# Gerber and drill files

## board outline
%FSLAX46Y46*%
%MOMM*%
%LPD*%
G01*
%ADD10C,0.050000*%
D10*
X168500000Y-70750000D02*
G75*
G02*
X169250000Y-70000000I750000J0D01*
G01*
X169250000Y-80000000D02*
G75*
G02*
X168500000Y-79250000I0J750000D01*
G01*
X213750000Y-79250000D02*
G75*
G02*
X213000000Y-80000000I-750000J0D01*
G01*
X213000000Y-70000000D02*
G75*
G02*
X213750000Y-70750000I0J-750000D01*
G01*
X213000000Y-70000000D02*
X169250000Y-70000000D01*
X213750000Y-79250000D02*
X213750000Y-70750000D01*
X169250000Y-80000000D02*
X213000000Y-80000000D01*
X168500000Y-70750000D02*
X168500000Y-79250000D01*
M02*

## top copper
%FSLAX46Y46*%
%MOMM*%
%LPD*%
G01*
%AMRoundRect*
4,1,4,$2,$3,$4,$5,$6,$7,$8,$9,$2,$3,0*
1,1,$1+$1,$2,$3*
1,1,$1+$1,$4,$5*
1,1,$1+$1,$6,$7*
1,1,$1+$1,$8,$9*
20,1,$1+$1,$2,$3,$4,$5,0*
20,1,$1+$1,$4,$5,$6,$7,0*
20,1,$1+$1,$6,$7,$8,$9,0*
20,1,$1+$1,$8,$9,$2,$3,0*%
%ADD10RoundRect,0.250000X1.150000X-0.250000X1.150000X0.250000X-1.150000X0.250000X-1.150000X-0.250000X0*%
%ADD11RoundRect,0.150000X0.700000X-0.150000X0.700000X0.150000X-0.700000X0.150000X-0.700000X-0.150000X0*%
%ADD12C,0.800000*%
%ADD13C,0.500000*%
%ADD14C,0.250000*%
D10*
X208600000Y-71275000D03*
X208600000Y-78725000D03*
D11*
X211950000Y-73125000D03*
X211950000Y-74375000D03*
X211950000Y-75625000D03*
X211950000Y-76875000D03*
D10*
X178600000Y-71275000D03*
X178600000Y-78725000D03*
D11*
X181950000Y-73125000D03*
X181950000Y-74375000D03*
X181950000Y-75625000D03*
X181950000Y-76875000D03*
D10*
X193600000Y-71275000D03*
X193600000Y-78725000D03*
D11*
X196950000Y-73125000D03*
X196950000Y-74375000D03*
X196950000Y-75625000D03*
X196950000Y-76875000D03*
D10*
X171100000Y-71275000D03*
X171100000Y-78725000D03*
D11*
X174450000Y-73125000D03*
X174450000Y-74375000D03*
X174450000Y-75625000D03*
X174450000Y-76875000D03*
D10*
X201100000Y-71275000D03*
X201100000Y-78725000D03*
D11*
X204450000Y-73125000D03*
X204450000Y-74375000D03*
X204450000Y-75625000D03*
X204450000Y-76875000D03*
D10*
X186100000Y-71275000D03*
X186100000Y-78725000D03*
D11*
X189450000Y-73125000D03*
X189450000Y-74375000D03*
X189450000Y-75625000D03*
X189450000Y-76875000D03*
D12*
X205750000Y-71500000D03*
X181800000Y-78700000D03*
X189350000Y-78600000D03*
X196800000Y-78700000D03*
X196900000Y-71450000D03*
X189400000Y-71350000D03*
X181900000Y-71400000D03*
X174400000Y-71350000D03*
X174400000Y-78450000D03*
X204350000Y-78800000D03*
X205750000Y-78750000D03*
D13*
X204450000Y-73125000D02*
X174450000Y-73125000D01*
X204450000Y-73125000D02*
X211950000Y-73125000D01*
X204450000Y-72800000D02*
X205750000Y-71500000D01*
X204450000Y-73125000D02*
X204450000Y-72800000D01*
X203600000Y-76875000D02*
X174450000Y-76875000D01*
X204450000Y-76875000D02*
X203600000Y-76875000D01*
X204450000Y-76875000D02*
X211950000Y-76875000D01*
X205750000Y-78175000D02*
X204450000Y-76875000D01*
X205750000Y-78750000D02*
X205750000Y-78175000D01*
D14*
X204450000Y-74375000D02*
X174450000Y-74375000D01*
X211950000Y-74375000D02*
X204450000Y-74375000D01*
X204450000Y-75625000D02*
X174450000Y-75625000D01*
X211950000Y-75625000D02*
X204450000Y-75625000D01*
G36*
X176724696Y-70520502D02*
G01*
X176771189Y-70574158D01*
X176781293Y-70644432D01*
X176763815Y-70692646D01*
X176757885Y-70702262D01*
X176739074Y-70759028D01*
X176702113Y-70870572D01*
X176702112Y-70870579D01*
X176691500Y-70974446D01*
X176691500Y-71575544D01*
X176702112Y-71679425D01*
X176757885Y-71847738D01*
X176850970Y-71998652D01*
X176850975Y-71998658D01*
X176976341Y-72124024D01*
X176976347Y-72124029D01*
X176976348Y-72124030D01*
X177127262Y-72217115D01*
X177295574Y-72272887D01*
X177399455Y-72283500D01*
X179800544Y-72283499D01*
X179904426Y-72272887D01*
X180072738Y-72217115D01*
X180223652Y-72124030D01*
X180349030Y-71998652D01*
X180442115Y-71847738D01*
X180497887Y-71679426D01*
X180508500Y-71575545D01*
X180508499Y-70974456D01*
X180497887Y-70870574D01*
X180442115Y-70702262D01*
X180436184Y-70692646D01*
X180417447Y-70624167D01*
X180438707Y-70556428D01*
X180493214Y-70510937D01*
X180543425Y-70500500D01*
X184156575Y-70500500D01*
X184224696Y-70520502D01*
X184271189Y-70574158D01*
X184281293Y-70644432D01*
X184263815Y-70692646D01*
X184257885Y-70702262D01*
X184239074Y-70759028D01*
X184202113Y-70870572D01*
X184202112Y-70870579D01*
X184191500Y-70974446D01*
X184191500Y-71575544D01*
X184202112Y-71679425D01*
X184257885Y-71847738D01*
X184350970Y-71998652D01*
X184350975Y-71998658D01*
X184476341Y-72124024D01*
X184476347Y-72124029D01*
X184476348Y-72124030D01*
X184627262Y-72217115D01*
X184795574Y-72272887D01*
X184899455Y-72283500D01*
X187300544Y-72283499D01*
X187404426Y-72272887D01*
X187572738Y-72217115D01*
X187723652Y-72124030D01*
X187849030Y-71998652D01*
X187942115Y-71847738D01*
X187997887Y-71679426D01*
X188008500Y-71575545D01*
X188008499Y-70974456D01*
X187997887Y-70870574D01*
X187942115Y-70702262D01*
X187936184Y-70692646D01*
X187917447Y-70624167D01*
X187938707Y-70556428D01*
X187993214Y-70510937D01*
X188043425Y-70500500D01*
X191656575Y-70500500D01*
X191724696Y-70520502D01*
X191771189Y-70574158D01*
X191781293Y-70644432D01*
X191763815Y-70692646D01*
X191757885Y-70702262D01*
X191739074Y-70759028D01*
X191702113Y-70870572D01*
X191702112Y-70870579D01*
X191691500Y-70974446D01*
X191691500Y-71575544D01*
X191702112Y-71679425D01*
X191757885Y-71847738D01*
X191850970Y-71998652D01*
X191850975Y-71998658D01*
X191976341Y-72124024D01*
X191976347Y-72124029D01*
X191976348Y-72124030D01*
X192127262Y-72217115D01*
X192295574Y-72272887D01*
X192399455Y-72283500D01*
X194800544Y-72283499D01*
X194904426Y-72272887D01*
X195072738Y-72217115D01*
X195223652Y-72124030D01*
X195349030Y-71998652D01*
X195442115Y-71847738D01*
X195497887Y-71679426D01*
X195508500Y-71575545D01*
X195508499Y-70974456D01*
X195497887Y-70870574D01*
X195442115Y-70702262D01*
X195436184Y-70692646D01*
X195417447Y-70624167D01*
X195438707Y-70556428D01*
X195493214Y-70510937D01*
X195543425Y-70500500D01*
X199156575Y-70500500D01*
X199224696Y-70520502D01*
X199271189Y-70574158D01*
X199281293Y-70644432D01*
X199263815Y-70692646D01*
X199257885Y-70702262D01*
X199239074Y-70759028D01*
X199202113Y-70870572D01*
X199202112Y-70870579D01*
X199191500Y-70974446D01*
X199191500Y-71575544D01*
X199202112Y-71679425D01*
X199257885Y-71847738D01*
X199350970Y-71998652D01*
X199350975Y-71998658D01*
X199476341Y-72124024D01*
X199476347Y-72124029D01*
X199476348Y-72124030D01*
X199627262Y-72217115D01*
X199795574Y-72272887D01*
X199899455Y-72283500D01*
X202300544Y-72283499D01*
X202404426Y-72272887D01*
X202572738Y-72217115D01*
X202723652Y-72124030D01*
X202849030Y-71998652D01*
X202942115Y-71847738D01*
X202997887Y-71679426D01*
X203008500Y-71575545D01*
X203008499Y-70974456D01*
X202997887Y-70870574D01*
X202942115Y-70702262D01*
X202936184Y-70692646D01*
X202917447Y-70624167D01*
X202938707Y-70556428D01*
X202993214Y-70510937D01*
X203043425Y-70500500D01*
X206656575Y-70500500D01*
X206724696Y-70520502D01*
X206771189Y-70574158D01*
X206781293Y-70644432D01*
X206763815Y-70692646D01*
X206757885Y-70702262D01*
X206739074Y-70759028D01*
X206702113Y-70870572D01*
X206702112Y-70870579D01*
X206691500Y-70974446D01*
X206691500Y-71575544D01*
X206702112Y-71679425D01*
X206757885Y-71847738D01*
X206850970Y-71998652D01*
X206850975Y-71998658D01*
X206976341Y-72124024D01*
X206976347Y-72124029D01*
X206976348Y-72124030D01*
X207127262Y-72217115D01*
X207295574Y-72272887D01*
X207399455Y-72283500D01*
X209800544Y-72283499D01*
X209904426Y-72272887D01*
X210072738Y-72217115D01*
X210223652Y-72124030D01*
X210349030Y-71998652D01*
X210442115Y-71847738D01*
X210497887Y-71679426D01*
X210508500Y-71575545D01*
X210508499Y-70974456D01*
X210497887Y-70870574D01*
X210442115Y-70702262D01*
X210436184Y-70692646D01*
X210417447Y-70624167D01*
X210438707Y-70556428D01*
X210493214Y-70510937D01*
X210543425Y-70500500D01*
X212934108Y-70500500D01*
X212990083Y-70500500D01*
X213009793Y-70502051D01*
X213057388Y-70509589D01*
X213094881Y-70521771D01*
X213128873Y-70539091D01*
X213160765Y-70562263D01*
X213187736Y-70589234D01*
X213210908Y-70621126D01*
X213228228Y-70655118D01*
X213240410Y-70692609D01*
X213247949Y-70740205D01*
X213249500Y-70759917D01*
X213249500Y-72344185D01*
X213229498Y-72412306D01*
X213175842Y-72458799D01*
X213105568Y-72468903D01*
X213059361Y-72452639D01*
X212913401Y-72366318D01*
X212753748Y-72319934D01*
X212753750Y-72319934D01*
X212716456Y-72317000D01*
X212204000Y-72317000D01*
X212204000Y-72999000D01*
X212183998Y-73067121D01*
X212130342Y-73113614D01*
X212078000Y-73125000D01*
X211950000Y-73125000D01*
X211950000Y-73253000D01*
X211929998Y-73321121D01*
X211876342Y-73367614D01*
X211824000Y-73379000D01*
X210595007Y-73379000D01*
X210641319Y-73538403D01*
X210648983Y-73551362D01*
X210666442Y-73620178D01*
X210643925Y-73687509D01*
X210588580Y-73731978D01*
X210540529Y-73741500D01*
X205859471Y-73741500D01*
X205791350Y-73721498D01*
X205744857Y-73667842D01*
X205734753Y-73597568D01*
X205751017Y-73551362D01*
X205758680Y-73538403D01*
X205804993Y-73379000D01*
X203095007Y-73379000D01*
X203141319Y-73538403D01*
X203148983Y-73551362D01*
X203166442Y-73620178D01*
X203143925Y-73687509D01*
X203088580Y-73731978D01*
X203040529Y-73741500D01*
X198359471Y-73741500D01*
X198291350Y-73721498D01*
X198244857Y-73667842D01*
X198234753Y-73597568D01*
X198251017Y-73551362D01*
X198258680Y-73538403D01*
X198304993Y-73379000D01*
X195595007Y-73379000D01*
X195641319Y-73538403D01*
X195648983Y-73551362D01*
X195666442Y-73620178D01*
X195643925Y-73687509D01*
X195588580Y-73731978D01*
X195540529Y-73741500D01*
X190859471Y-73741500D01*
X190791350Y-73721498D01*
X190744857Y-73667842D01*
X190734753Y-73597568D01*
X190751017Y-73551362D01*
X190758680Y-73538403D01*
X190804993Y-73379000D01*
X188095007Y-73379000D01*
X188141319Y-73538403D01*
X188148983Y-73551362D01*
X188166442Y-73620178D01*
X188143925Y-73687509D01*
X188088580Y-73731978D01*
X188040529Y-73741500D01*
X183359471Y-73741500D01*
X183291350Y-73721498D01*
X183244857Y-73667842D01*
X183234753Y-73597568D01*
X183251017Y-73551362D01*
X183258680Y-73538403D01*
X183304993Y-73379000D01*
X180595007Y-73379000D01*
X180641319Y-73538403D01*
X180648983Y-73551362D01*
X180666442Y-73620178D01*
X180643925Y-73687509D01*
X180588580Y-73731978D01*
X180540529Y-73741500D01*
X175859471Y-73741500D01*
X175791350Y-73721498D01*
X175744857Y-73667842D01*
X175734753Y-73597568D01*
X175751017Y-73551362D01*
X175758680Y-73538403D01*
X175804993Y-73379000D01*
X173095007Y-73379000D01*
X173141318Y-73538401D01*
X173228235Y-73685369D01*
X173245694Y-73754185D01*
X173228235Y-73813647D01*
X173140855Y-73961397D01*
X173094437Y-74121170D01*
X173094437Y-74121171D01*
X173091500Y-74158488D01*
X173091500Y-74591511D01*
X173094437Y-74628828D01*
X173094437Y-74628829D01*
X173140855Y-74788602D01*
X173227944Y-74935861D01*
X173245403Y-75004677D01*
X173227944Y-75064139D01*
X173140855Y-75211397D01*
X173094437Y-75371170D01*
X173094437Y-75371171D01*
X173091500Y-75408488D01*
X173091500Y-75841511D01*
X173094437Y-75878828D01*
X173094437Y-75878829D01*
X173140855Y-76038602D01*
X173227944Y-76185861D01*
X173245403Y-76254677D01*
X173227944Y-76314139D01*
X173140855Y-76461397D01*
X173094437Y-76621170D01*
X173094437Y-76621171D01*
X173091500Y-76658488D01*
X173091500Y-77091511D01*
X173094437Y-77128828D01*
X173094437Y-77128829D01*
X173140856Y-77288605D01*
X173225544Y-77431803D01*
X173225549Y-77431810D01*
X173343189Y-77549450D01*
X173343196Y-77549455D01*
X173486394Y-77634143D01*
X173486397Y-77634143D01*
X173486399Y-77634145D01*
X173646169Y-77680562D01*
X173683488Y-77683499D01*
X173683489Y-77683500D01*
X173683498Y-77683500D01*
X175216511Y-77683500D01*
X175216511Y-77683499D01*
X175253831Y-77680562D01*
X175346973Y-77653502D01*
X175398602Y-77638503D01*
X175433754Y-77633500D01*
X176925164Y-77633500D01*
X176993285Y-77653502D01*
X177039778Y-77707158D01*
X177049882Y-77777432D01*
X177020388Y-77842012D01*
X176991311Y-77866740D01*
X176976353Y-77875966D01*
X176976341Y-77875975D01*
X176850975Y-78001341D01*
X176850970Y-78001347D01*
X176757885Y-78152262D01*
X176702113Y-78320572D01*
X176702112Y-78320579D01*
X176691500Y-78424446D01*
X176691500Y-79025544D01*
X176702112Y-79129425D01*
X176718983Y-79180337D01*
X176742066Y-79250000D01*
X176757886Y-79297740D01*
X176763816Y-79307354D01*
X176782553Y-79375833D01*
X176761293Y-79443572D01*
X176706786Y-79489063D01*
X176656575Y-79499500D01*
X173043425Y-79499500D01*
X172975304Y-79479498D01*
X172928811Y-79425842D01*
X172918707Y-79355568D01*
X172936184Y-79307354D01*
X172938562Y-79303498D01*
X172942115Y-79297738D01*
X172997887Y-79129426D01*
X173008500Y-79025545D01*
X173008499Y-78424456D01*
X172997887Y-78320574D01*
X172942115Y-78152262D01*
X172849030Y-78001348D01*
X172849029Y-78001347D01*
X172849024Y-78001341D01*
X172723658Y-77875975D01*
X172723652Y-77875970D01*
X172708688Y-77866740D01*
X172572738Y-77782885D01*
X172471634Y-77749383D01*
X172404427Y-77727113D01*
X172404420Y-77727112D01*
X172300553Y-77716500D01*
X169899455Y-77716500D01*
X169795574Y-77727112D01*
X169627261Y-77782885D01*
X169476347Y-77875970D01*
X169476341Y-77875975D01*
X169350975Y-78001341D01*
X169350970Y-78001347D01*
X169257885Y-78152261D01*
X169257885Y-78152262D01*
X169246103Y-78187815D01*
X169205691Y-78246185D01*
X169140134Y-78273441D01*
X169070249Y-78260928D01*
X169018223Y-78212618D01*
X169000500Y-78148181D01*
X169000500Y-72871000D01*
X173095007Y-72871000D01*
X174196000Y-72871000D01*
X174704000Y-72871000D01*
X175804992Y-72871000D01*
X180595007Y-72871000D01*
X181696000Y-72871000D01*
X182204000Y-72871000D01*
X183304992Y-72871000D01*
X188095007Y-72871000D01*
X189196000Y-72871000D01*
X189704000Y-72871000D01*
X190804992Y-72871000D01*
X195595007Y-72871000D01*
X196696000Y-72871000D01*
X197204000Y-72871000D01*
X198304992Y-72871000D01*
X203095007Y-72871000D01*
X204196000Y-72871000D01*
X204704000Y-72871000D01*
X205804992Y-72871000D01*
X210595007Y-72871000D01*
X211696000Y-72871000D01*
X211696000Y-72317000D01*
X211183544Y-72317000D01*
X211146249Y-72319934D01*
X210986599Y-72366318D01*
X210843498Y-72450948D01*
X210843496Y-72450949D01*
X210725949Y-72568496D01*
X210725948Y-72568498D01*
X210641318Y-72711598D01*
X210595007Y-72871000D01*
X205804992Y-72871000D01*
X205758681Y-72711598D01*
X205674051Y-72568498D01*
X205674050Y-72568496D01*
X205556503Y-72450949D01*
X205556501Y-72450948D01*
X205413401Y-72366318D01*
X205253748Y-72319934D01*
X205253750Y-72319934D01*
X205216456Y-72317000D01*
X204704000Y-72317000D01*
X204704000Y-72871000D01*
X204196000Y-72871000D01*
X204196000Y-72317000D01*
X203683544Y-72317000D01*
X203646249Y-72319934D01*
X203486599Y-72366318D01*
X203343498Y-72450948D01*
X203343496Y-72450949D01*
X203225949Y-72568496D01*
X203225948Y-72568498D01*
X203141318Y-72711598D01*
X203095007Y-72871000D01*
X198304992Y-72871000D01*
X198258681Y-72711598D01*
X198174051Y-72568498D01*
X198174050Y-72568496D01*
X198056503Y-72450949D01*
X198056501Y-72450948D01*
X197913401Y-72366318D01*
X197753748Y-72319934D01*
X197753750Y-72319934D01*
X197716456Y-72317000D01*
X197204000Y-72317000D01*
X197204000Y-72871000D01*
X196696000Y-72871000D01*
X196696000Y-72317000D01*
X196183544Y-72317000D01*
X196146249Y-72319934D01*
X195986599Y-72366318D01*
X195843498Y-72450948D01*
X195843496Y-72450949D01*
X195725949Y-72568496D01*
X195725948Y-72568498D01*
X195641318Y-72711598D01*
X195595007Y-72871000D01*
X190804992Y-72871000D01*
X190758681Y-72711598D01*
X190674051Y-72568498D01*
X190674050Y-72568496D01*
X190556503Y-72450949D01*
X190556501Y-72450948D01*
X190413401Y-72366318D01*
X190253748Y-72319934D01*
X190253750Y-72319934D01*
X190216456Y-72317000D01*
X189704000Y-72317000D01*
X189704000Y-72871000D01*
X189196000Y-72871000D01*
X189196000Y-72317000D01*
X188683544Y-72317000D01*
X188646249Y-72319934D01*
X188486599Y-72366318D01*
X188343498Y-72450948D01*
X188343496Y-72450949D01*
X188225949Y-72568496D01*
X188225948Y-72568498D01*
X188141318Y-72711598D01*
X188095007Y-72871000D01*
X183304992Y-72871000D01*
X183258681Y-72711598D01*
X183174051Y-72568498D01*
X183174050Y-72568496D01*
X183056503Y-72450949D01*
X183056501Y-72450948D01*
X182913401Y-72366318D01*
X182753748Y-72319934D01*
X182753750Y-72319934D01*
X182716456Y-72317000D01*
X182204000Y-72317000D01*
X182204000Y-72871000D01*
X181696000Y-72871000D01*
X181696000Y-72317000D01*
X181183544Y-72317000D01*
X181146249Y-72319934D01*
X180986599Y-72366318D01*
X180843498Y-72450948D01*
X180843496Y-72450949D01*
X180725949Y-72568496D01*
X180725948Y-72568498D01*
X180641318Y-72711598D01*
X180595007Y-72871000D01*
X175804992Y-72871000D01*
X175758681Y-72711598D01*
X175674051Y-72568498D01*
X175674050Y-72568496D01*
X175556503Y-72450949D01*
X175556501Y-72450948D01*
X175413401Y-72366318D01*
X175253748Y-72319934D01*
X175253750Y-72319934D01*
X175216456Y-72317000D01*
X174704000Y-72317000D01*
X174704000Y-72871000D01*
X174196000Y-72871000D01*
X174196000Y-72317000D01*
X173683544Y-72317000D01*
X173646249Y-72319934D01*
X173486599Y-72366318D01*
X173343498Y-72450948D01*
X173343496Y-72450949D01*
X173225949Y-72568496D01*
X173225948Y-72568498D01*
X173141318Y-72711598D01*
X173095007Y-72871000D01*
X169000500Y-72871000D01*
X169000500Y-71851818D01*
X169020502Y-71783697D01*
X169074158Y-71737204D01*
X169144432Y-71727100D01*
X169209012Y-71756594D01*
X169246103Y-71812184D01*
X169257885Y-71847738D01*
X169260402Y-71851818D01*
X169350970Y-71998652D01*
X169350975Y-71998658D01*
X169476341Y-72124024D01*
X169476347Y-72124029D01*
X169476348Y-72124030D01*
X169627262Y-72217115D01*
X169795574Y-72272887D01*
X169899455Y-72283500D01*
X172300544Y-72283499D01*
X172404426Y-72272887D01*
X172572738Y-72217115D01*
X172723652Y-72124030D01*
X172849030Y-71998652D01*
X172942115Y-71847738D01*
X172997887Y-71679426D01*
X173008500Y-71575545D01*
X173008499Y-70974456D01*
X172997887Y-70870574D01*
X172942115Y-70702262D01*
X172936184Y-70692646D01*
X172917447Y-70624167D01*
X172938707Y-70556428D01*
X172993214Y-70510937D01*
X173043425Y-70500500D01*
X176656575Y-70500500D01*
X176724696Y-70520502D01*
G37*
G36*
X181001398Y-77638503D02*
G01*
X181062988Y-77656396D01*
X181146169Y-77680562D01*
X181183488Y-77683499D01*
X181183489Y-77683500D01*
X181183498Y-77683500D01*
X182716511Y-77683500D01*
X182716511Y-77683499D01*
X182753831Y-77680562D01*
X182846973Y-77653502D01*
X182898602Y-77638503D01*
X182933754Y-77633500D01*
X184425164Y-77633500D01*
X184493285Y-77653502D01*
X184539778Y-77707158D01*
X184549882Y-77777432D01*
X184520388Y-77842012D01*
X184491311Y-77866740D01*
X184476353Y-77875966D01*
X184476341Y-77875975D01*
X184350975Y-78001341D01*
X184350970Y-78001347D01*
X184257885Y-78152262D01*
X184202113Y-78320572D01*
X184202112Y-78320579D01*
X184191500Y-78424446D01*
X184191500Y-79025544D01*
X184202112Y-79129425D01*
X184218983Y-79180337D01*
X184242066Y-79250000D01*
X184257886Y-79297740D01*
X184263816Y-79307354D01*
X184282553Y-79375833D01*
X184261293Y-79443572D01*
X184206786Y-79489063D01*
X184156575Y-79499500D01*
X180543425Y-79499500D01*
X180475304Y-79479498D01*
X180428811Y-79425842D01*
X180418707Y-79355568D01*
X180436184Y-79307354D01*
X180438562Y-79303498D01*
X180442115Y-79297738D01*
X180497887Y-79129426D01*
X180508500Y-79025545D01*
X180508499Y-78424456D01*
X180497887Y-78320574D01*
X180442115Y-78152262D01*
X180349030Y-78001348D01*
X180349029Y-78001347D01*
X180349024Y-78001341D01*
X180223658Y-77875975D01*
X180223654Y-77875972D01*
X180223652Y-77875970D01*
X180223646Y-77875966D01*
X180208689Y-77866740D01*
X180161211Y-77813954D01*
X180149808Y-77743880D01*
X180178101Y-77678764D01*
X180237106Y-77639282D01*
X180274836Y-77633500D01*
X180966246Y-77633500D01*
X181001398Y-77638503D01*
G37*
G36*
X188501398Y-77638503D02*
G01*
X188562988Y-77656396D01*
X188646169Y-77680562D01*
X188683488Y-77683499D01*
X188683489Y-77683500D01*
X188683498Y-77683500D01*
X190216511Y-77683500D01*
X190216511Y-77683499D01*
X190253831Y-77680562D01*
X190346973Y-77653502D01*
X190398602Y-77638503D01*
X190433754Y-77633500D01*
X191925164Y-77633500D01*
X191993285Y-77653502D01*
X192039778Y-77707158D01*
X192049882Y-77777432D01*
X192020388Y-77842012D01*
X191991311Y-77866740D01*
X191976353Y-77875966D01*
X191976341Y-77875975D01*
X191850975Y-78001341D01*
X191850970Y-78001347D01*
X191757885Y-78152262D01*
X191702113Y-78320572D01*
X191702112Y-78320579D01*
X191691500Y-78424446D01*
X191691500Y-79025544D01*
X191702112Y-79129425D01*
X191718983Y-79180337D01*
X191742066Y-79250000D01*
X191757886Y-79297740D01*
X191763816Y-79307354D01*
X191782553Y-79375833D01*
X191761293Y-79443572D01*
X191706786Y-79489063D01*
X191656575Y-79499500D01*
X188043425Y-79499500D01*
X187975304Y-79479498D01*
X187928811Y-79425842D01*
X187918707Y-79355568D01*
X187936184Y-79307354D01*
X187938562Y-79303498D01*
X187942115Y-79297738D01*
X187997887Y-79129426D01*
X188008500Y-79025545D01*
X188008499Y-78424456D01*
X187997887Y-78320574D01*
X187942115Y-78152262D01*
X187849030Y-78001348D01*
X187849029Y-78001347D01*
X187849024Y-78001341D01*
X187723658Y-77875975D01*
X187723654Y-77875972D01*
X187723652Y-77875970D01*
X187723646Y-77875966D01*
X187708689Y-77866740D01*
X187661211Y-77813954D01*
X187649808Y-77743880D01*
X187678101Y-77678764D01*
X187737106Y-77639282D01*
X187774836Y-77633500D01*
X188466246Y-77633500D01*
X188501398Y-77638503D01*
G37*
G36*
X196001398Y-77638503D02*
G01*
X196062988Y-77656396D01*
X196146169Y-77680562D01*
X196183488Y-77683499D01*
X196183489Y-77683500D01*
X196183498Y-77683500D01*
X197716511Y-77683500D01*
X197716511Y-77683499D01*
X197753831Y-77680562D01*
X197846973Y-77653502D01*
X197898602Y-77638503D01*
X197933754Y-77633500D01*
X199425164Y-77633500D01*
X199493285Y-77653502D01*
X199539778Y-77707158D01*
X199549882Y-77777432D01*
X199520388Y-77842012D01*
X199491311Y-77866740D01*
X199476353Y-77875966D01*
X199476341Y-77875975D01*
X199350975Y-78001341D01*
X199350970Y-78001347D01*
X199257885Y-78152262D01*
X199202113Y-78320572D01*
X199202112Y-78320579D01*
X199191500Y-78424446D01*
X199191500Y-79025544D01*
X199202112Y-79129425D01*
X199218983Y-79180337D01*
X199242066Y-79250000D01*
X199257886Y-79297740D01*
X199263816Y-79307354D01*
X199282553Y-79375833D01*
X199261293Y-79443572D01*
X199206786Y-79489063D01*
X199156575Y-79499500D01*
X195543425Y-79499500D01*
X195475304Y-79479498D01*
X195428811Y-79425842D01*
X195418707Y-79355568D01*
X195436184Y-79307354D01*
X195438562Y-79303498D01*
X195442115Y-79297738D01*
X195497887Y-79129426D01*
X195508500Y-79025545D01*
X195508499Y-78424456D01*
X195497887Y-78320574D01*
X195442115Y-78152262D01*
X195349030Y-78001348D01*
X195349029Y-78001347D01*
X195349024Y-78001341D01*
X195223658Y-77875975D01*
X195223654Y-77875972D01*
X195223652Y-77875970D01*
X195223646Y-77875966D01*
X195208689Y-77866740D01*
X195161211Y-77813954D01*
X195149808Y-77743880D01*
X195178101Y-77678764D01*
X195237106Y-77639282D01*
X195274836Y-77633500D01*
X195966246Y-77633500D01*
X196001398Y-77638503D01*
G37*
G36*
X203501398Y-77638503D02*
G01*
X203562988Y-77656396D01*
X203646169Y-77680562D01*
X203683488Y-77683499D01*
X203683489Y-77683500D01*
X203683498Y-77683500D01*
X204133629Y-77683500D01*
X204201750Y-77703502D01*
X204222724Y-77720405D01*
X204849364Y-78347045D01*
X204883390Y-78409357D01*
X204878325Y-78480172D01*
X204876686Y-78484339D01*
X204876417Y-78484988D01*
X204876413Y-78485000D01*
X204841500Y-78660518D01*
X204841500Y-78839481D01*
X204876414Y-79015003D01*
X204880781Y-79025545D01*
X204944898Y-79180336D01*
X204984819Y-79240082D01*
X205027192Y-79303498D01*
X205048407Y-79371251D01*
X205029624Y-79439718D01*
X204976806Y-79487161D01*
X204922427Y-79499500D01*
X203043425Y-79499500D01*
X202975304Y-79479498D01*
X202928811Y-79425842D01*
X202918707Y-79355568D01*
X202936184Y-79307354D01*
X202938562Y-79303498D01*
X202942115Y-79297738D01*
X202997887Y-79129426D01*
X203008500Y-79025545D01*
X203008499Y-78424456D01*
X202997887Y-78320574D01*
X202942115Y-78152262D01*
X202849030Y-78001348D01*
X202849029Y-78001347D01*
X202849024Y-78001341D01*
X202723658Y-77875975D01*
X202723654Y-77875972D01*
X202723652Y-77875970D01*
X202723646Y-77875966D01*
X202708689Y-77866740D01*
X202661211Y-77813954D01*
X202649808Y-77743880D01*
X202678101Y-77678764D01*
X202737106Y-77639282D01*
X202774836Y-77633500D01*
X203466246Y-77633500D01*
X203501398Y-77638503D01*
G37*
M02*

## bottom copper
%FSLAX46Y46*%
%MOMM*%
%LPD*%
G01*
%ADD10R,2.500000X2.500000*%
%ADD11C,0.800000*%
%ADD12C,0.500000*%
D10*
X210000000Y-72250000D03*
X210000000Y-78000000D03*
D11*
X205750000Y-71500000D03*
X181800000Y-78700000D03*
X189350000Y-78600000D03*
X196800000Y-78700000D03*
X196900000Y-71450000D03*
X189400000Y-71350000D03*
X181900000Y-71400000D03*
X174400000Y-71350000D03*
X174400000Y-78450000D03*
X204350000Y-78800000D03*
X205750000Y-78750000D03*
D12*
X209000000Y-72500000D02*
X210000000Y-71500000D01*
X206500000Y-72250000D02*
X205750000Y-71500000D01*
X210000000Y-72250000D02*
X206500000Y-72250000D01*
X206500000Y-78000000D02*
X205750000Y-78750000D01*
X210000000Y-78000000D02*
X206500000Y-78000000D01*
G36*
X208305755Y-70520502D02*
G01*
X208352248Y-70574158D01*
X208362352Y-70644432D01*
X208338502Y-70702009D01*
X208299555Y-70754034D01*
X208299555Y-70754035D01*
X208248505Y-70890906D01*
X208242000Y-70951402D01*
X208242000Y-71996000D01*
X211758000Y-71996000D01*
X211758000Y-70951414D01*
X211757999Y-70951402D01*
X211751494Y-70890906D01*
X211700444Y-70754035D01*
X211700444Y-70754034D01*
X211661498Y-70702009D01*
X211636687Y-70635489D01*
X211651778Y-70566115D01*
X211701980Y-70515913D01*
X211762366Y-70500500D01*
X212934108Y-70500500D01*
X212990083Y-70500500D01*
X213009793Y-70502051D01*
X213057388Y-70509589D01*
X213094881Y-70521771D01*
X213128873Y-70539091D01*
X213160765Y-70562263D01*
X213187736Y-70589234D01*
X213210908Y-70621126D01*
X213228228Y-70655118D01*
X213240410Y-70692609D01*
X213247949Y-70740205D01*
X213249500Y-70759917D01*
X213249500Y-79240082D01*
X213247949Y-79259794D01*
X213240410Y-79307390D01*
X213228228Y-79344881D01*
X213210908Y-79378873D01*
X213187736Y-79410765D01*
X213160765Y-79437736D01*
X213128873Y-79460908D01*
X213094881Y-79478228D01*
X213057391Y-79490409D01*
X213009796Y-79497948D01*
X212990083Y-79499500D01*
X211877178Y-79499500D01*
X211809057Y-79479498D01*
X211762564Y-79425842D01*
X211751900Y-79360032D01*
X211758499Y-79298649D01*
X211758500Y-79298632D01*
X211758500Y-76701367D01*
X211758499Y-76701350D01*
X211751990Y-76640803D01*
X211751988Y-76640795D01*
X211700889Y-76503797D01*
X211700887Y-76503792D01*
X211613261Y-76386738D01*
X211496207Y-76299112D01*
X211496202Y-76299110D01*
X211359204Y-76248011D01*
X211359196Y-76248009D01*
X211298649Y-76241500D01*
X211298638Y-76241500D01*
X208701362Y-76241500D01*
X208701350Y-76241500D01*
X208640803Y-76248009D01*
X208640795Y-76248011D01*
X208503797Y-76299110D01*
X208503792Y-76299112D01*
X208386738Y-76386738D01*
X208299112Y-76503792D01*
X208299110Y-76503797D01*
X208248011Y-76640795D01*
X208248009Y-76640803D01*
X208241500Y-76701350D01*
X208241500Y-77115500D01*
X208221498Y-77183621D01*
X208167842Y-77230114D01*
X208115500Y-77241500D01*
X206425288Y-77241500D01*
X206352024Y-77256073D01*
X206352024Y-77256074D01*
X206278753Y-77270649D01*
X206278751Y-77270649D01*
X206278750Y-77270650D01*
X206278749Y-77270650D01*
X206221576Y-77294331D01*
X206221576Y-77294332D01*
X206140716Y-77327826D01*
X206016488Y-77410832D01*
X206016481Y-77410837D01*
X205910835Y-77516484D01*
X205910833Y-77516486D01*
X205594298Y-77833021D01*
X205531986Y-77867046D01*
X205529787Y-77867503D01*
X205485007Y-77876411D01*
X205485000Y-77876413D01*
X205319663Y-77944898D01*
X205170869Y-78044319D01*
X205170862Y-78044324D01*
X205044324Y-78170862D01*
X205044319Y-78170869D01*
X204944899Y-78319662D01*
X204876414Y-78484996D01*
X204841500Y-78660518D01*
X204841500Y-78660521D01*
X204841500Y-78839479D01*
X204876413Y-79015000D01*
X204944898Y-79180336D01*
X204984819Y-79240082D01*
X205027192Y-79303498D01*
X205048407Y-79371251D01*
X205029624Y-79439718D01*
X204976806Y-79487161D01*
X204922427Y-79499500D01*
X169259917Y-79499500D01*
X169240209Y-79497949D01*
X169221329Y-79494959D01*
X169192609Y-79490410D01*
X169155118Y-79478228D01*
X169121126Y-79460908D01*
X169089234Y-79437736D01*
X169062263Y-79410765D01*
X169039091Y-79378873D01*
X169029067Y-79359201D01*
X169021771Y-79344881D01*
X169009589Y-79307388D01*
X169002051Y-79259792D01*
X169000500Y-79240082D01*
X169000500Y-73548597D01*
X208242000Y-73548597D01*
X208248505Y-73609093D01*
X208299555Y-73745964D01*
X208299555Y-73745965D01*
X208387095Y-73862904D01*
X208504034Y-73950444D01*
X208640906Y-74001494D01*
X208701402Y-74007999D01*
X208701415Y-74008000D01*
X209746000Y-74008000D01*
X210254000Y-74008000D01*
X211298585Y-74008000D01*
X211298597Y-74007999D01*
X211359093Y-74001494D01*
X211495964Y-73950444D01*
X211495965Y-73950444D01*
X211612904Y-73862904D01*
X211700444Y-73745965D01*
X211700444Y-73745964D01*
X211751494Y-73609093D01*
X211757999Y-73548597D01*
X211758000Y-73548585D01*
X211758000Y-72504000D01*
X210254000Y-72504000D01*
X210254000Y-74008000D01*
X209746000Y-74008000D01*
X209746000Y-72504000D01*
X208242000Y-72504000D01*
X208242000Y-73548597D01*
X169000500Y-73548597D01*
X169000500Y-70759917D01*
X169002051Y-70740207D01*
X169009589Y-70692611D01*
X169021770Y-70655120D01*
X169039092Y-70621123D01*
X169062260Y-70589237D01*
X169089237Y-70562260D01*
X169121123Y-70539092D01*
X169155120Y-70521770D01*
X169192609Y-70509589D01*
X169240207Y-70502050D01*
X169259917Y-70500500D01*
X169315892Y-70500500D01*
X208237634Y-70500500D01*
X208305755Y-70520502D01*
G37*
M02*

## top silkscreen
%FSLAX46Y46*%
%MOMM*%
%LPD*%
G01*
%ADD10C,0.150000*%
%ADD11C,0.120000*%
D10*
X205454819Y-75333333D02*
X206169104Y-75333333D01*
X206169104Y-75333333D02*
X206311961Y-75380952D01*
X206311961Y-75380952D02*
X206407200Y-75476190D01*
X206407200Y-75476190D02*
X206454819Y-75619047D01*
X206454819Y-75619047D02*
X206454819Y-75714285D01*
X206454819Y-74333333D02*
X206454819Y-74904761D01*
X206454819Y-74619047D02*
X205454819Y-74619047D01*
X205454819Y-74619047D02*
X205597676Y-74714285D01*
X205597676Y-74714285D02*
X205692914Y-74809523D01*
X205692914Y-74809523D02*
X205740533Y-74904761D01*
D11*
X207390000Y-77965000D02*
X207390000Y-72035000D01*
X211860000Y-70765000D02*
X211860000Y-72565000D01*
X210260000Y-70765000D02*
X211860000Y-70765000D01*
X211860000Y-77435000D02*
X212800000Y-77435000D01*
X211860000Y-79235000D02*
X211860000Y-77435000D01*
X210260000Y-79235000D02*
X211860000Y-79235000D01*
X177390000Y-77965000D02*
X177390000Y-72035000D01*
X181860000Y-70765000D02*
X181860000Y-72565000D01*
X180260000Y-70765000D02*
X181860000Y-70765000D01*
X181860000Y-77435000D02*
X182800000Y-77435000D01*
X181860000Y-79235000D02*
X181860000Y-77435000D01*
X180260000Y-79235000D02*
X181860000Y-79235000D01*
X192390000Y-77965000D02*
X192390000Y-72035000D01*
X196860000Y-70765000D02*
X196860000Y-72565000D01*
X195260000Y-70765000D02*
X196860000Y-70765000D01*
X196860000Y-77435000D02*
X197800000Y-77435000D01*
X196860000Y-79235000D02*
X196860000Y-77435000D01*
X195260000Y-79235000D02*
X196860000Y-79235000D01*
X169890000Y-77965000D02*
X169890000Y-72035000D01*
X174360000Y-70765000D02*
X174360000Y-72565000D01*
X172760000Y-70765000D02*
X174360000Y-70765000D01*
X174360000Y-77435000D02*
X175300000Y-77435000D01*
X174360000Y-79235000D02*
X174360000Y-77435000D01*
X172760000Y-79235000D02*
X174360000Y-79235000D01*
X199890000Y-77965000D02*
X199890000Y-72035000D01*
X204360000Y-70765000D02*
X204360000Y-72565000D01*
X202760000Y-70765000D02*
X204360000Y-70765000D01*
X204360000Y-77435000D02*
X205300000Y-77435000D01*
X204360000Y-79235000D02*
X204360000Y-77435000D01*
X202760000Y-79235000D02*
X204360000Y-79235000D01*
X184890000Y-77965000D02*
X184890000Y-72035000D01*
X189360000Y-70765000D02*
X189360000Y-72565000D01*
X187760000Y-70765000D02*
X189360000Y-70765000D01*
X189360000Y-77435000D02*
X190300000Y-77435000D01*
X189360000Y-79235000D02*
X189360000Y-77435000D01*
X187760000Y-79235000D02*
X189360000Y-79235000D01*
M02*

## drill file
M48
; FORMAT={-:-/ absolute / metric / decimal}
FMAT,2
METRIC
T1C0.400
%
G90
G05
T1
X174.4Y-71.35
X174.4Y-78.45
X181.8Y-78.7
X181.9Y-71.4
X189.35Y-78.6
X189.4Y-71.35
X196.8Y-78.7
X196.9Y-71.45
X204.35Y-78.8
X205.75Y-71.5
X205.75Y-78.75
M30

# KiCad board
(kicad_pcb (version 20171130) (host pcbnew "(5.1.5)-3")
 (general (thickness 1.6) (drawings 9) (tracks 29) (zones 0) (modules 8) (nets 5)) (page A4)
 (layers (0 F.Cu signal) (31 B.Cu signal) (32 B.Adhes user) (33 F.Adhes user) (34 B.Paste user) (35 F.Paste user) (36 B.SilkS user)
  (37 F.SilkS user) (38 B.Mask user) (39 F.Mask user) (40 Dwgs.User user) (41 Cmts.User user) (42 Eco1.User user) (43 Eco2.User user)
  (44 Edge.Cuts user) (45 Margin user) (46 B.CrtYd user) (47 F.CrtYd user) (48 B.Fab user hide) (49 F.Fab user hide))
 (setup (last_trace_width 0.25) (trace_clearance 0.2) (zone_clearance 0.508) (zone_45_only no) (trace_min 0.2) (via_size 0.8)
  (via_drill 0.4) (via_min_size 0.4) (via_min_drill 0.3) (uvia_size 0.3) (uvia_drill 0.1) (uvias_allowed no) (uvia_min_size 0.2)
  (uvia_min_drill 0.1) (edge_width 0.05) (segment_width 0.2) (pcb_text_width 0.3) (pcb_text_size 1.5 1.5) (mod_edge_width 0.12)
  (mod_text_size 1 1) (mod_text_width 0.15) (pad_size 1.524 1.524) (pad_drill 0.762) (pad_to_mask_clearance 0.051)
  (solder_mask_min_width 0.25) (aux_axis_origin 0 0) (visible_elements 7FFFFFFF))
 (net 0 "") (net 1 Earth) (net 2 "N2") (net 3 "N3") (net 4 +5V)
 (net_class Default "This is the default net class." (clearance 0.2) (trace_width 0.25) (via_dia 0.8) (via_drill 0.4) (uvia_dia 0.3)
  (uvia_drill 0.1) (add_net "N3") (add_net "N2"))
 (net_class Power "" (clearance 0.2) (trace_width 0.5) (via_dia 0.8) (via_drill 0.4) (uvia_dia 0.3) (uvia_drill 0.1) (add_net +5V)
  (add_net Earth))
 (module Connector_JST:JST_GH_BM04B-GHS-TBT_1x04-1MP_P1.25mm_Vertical (layer F.Cu) (at 210 75 90)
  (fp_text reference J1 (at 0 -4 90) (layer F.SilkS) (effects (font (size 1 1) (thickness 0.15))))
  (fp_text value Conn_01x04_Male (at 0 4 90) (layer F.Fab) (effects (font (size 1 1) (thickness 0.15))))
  (fp_line (start -2.965 -2.61) (end 2.965 -2.61) (layer F.SilkS) (width 0.12))
  (fp_line (start 4.235 1.86) (end 2.435 1.86) (layer F.SilkS) (width 0.12))
  (fp_line (start 4.235 0.26) (end 4.235 1.86) (layer F.SilkS) (width 0.12))
  (fp_line (start -2.435 1.86) (end -2.435 2.8) (layer F.SilkS) (width 0.12))
  (fp_line (start -4.235 1.86) (end -2.435 1.86) (layer F.SilkS) (width 0.12))
  (fp_line (start -4.235 0.26) (end -4.235 1.86) (layer F.SilkS) (width 0.12))
  (pad MP smd roundrect (at 3.725 -1.4 90) (size 1 2.8) (layers F.Cu F.Paste F.Mask) (roundrect_rratio 0.25))
  (pad MP smd roundrect (at -3.725 -1.4 90) (size 1 2.8) (layers F.Cu F.Paste F.Mask) (roundrect_rratio 0.25))
  (pad 4 smd roundrect (at 1.875 1.95 90) (size 0.6 1.7) (layers F.Cu F.Paste F.Mask) (roundrect_rratio 0.25) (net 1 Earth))
  (pad 3 smd roundrect (at 0.625 1.95 90) (size 0.6 1.7) (layers F.Cu F.Paste F.Mask) (roundrect_rratio 0.25) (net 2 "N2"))
  (pad 2 smd roundrect (at -0.625 1.95 90) (size 0.6 1.7) (layers F.Cu F.Paste F.Mask) (roundrect_rratio 0.25) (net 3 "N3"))
  (pad 1 smd roundrect (at -1.875 1.95 90) (size 0.6 1.7) (layers F.Cu F.Paste F.Mask) (roundrect_rratio 0.25) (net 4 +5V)))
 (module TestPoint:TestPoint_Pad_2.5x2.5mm (layer B.Cu) (at 210 72.25)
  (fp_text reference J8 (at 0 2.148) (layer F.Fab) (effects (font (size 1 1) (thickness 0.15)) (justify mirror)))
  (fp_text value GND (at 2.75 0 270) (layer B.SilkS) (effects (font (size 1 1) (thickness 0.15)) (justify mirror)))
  (pad 1 smd rect (at 0 0) (size 2.5 2.5) (layers B.Cu B.Mask) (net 1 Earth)))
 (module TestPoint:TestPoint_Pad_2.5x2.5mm (layer B.Cu) (at 210 78)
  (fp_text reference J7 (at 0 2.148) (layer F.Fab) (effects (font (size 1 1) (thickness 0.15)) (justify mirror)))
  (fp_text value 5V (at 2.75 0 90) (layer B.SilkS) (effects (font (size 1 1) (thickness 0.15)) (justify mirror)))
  (pad 1 smd rect (at 0 0) (size 2.5 2.5) (layers B.Cu B.Mask) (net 4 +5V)))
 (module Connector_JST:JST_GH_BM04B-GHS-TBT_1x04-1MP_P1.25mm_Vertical (layer F.Cu) (at 180 75 90)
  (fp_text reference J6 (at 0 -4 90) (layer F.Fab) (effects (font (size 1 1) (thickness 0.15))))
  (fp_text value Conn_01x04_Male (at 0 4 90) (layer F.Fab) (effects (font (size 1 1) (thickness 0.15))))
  (fp_line (start -2.965 -2.61) (end 2.965 -2.61) (layer F.SilkS) (width 0.12))
  (fp_line (start 4.235 1.86) (end 2.435 1.86) (layer F.SilkS) (width 0.12))
  (fp_line (start 4.235 0.26) (end 4.235 1.86) (layer F.SilkS) (width 0.12))
  (fp_line (start -2.435 1.86) (end -2.435 2.8) (layer F.SilkS) (width 0.12))
  (fp_line (start -4.235 1.86) (end -2.435 1.86) (layer F.SilkS) (width 0.12))
  (fp_line (start -4.235 0.26) (end -4.235 1.86) (layer F.SilkS) (width 0.12))
  (pad MP smd roundrect (at 3.725 -1.4 90) (size 1 2.8) (layers F.Cu F.Paste F.Mask) (roundrect_rratio 0.25))
  (pad MP smd roundrect (at -3.725 -1.4 90) (size 1 2.8) (layers F.Cu F.Paste F.Mask) (roundrect_rratio 0.25))
  (pad 4 smd roundrect (at 1.875 1.95 90) (size 0.6 1.7) (layers F.Cu F.Paste F.Mask) (roundrect_rratio 0.25) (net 1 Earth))
  (pad 3 smd roundrect (at 0.625 1.95 90) (size 0.6 1.7) (layers F.Cu F.Paste F.Mask) (roundrect_rratio 0.25) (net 2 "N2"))
  (pad 2 smd roundrect (at -0.625 1.95 90) (size 0.6 1.7) (layers F.Cu F.Paste F.Mask) (roundrect_rratio 0.25) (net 3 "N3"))
  (pad 1 smd roundrect (at -1.875 1.95 90) (size 0.6 1.7) (layers F.Cu F.Paste F.Mask) (roundrect_rratio 0.25) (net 4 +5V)))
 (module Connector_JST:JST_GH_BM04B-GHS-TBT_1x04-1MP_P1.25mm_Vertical (layer F.Cu) (at 195 75 90)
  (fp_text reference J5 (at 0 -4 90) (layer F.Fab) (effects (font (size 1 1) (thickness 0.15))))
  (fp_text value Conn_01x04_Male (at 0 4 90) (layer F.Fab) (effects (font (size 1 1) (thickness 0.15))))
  (fp_line (start -2.965 -2.61) (end 2.965 -2.61) (layer F.SilkS) (width 0.12))
  (fp_line (start 4.235 1.86) (end 2.435 1.86) (layer F.SilkS) (width 0.12))
  (fp_line (start 4.235 0.26) (end 4.235 1.86) (layer F.SilkS) (width 0.12))
  (fp_line (start -2.435 1.86) (end -2.435 2.8) (layer F.SilkS) (width 0.12))
  (fp_line (start -4.235 1.86) (end -2.435 1.86) (layer F.SilkS) (width 0.12))
  (fp_line (start -4.235 0.26) (end -4.235 1.86) (layer F.SilkS) (width 0.12))
  (pad MP smd roundrect (at 3.725 -1.4 90) (size 1 2.8) (layers F.Cu F.Paste F.Mask) (roundrect_rratio 0.25))
  (pad MP smd roundrect (at -3.725 -1.4 90) (size 1 2.8) (layers F.Cu F.Paste F.Mask) (roundrect_rratio 0.25))
  (pad 4 smd roundrect (at 1.875 1.95 90) (size 0.6 1.7) (layers F.Cu F.Paste F.Mask) (roundrect_rratio 0.25) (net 1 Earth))
  (pad 3 smd roundrect (at 0.625 1.95 90) (size 0.6 1.7) (layers F.Cu F.Paste F.Mask) (roundrect_rratio 0.25) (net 2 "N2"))
  (pad 2 smd roundrect (at -0.625 1.95 90) (size 0.6 1.7) (layers F.Cu F.Paste F.Mask) (roundrect_rratio 0.25) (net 3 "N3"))
  (pad 1 smd roundrect (at -1.875 1.95 90) (size 0.6 1.7) (layers F.Cu F.Paste F.Mask) (roundrect_rratio 0.25) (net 4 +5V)))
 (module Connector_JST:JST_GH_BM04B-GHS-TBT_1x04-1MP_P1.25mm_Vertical (layer F.Cu) (at 172.5 75 90)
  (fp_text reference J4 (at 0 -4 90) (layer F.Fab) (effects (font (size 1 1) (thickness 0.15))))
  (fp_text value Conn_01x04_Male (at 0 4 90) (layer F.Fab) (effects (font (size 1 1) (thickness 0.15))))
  (fp_line (start -2.965 -2.61) (end 2.965 -2.61) (layer F.SilkS) (width 0.12))
  (fp_line (start 4.235 1.86) (end 2.435 1.86) (layer F.SilkS) (width 0.12))
  (fp_line (start 4.235 0.26) (end 4.235 1.86) (layer F.SilkS) (width 0.12))
  (fp_line (start -2.435 1.86) (end -2.435 2.8) (layer F.SilkS) (width 0.12))
  (fp_line (start -4.235 1.86) (end -2.435 1.86) (layer F.SilkS) (width 0.12))
  (fp_line (start -4.235 0.26) (end -4.235 1.86) (layer F.SilkS) (width 0.12))
  (pad MP smd roundrect (at 3.725 -1.4 90) (size 1 2.8) (layers F.Cu F.Paste F.Mask) (roundrect_rratio 0.25))
  (pad MP smd roundrect (at -3.725 -1.4 90) (size 1 2.8) (layers F.Cu F.Paste F.Mask) (roundrect_rratio 0.25))
  (pad 4 smd roundrect (at 1.875 1.95 90) (size 0.6 1.7) (layers F.Cu F.Paste F.Mask) (roundrect_rratio 0.25) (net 1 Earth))
  (pad 3 smd roundrect (at 0.625 1.95 90) (size 0.6 1.7) (layers F.Cu F.Paste F.Mask) (roundrect_rratio 0.25) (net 2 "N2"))
  (pad 2 smd roundrect (at -0.625 1.95 90) (size 0.6 1.7) (layers F.Cu F.Paste F.Mask) (roundrect_rratio 0.25) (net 3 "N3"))
  (pad 1 smd roundrect (at -1.875 1.95 90) (size 0.6 1.7) (layers F.Cu F.Paste F.Mask) (roundrect_rratio 0.25) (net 4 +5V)))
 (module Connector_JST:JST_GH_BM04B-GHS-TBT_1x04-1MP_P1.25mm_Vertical (layer F.Cu) (at 202.5 75 90)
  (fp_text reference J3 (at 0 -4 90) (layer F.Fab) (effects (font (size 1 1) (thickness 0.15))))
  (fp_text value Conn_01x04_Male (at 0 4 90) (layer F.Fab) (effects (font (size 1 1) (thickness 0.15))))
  (fp_line (start -2.965 -2.61) (end 2.965 -2.61) (layer F.SilkS) (width 0.12))
  (fp_line (start 4.235 1.86) (end 2.435 1.86) (layer F.SilkS) (width 0.12))
  (fp_line (start 4.235 0.26) (end 4.235 1.86) (layer F.SilkS) (width 0.12))
  (fp_line (start -2.435 1.86) (end -2.435 2.8) (layer F.SilkS) (width 0.12))
  (fp_line (start -4.235 1.86) (end -2.435 1.86) (layer F.SilkS) (width 0.12))
  (fp_line (start -4.235 0.26) (end -4.235 1.86) (layer F.SilkS) (width 0.12))
  (pad MP smd roundrect (at 3.725 -1.4 90) (size 1 2.8) (layers F.Cu F.Paste F.Mask) (roundrect_rratio 0.25))
  (pad MP smd roundrect (at -3.725 -1.4 90) (size 1 2.8) (layers F.Cu F.Paste F.Mask) (roundrect_rratio 0.25))
  (pad 4 smd roundrect (at 1.875 1.95 90) (size 0.6 1.7) (layers F.Cu F.Paste F.Mask) (roundrect_rratio 0.25) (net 1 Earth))
  (pad 3 smd roundrect (at 0.625 1.95 90) (size 0.6 1.7) (layers F.Cu F.Paste F.Mask) (roundrect_rratio 0.25) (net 2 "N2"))
  (pad 2 smd roundrect (at -0.625 1.95 90) (size 0.6 1.7) (layers F.Cu F.Paste F.Mask) (roundrect_rratio 0.25) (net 3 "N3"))
  (pad 1 smd roundrect (at -1.875 1.95 90) (size 0.6 1.7) (layers F.Cu F.Paste F.Mask) (roundrect_rratio 0.25) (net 4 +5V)))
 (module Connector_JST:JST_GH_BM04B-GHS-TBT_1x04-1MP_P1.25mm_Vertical (layer F.Cu) (at 187.5 75 90)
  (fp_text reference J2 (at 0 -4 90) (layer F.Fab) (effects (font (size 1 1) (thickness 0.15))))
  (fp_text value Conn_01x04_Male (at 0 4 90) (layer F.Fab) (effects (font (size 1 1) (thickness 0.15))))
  (fp_line (start -2.965 -2.61) (end 2.965 -2.61) (layer F.SilkS) (width 0.12))
  (fp_line (start 4.235 1.86) (end 2.435 1.86) (layer F.SilkS) (width 0.12))
  (fp_line (start 4.235 0.26) (end 4.235 1.86) (layer F.SilkS) (width 0.12))
  (fp_line (start -2.435 1.86) (end -2.435 2.8) (layer F.SilkS) (width 0.12))
  (fp_line (start -4.235 1.86) (end -2.435 1.86) (layer F.SilkS) (width 0.12))
  (fp_line (start -4.235 0.26) (end -4.235 1.86) (layer F.SilkS) (width 0.12))
  (pad MP smd roundrect (at 3.725 -1.4 90) (size 1 2.8) (layers F.Cu F.Paste F.Mask) (roundrect_rratio 0.25))
  (pad MP smd roundrect (at -3.725 -1.4 90) (size 1 2.8) (layers F.Cu F.Paste F.Mask) (roundrect_rratio 0.25))
  (pad 4 smd roundrect (at 1.875 1.95 90) (size 0.6 1.7) (layers F.Cu F.Paste F.Mask) (roundrect_rratio 0.25) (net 1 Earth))
  (pad 3 smd roundrect (at 0.625 1.95 90) (size 0.6 1.7) (layers F.Cu F.Paste F.Mask) (roundrect_rratio 0.25) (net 2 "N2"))
  (pad 2 smd roundrect (at -0.625 1.95 90) (size 0.6 1.7) (layers F.Cu F.Paste F.Mask) (roundrect_rratio 0.25) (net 3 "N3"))
  (pad 1 smd roundrect (at -1.875 1.95 90) (size 0.6 1.7) (layers F.Cu F.Paste F.Mask) (roundrect_rratio 0.25) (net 4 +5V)))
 (gr_arc (start 169.25 70.75) (end 169.25 70) (angle -90) (layer Edge.Cuts) (width 0.05))
 (gr_arc (start 169.25 79.25) (end 168.5 79.25) (angle -90) (layer Edge.Cuts) (width 0.05))
 (gr_arc (start 213 79.25) (end 213 80) (angle -90) (layer Edge.Cuts) (width 0.05))
 (gr_arc (start 213 70.75) (end 213.75 70.75) (angle -90) (layer Edge.Cuts) (width 0.05))
 (gr_line (start 213 70) (end 169.25 70) (layer Edge.Cuts) (width 0.05))
 (gr_line (start 213.75 79.25) (end 213.75 70.75) (layer Edge.Cuts) (width 0.05))
 (gr_line (start 169.25 80) (end 213 80) (layer Edge.Cuts) (width 0.05))
 (gr_line (start 168.5 70.75) (end 168.5 79.25) (layer Edge.Cuts) (width 0.05))
 (segment (start 209 72.5) (end 210 71.5) (width 0.5) (layer B.Cu) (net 1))
 (segment (start 204.45 73.125) (end 174.45 73.125) (width 0.5) (layer F.Cu) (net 1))
 (via (at 205.75 71.5) (size 0.8) (drill 0.4) (layers F.Cu B.Cu) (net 1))
 (segment (start 204.45 73.125) (end 211.95 73.125) (width 0.5) (layer F.Cu) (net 1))
 (segment (start 204.45 72.8) (end 205.75 71.5) (width 0.5) (layer F.Cu) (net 1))
 (segment (start 204.45 73.125) (end 204.45 72.8) (width 0.5) (layer F.Cu) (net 1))
 (segment (start 206.5 72.25) (end 205.75 71.5) (width 0.5) (layer B.Cu) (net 1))
 (segment (start 210 72.25) (end 206.5 72.25) (width 0.5) (layer B.Cu) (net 1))
 (via (at 181.8 78.7) (size 0.8) (drill 0.4) (layers F.Cu B.Cu) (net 1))
 (via (at 189.35 78.6) (size 0.8) (drill 0.4) (layers F.Cu B.Cu) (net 1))
 (via (at 196.8 78.7) (size 0.8) (drill 0.4) (layers F.Cu B.Cu) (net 1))
 (via (at 196.9 71.45) (size 0.8) (drill 0.4) (layers F.Cu B.Cu) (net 1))
 (via (at 189.4 71.35) (size 0.8) (drill 0.4) (layers F.Cu B.Cu) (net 1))
 (via (at 181.9 71.4) (size 0.8) (drill 0.4) (layers F.Cu B.Cu) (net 1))
 (via (at 174.4 71.35) (size 0.8) (drill 0.4) (layers F.Cu B.Cu) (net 1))
 (via (at 174.4 78.45) (size 0.8) (drill 0.4) (layers F.Cu B.Cu) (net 1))
 (via (at 204.35 78.8) (size 0.8) (drill 0.4) (layers F.Cu B.Cu) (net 1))
 (via (at 205.75 78.75) (size 0.8) (drill 0.4) (layers F.Cu B.Cu) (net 4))
 (segment (start 203.6 76.875) (end 174.45 76.875) (width 0.5) (layer F.Cu) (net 4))
 (segment (start 204.45 76.875) (end 203.6 76.875) (width 0.5) (layer F.Cu) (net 4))
 (segment (start 204.45 76.875) (end 211.95 76.875) (width 0.5) (layer F.Cu) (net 4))
 (segment (start 205.75 78.175) (end 204.45 76.875) (width 0.5) (layer F.Cu) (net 4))
 (segment (start 205.75 78.75) (end 205.75 78.175) (width 0.5) (layer F.Cu) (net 4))
 (segment (start 206.5 78) (end 205.75 78.75) (width 0.5) (layer B.Cu) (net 4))
 (segment (start 210 78) (end 206.5 78) (width 0.5) (layer B.Cu) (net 4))
 (segment (start 204.45 74.375) (end 174.45 74.375) (width 0.25) (layer F.Cu) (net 2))
 (segment (start 211.95 74.375) (end 204.45 74.375) (width 0.25) (layer F.Cu) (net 2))
 (segment (start 204.45 75.625) (end 174.45 75.625) (width 0.25) (layer F.Cu) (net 3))
 (segment (start 211.95 75.625) (end 204.45 75.625) (width 0.25) (layer F.Cu) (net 3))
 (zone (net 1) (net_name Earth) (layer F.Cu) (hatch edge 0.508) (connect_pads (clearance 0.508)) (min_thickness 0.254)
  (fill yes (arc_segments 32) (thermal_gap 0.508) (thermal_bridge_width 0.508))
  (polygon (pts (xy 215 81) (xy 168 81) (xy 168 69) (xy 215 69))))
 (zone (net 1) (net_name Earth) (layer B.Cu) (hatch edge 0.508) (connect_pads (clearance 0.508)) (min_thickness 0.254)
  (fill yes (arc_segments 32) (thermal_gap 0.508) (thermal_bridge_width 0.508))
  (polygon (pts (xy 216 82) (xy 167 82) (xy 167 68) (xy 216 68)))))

